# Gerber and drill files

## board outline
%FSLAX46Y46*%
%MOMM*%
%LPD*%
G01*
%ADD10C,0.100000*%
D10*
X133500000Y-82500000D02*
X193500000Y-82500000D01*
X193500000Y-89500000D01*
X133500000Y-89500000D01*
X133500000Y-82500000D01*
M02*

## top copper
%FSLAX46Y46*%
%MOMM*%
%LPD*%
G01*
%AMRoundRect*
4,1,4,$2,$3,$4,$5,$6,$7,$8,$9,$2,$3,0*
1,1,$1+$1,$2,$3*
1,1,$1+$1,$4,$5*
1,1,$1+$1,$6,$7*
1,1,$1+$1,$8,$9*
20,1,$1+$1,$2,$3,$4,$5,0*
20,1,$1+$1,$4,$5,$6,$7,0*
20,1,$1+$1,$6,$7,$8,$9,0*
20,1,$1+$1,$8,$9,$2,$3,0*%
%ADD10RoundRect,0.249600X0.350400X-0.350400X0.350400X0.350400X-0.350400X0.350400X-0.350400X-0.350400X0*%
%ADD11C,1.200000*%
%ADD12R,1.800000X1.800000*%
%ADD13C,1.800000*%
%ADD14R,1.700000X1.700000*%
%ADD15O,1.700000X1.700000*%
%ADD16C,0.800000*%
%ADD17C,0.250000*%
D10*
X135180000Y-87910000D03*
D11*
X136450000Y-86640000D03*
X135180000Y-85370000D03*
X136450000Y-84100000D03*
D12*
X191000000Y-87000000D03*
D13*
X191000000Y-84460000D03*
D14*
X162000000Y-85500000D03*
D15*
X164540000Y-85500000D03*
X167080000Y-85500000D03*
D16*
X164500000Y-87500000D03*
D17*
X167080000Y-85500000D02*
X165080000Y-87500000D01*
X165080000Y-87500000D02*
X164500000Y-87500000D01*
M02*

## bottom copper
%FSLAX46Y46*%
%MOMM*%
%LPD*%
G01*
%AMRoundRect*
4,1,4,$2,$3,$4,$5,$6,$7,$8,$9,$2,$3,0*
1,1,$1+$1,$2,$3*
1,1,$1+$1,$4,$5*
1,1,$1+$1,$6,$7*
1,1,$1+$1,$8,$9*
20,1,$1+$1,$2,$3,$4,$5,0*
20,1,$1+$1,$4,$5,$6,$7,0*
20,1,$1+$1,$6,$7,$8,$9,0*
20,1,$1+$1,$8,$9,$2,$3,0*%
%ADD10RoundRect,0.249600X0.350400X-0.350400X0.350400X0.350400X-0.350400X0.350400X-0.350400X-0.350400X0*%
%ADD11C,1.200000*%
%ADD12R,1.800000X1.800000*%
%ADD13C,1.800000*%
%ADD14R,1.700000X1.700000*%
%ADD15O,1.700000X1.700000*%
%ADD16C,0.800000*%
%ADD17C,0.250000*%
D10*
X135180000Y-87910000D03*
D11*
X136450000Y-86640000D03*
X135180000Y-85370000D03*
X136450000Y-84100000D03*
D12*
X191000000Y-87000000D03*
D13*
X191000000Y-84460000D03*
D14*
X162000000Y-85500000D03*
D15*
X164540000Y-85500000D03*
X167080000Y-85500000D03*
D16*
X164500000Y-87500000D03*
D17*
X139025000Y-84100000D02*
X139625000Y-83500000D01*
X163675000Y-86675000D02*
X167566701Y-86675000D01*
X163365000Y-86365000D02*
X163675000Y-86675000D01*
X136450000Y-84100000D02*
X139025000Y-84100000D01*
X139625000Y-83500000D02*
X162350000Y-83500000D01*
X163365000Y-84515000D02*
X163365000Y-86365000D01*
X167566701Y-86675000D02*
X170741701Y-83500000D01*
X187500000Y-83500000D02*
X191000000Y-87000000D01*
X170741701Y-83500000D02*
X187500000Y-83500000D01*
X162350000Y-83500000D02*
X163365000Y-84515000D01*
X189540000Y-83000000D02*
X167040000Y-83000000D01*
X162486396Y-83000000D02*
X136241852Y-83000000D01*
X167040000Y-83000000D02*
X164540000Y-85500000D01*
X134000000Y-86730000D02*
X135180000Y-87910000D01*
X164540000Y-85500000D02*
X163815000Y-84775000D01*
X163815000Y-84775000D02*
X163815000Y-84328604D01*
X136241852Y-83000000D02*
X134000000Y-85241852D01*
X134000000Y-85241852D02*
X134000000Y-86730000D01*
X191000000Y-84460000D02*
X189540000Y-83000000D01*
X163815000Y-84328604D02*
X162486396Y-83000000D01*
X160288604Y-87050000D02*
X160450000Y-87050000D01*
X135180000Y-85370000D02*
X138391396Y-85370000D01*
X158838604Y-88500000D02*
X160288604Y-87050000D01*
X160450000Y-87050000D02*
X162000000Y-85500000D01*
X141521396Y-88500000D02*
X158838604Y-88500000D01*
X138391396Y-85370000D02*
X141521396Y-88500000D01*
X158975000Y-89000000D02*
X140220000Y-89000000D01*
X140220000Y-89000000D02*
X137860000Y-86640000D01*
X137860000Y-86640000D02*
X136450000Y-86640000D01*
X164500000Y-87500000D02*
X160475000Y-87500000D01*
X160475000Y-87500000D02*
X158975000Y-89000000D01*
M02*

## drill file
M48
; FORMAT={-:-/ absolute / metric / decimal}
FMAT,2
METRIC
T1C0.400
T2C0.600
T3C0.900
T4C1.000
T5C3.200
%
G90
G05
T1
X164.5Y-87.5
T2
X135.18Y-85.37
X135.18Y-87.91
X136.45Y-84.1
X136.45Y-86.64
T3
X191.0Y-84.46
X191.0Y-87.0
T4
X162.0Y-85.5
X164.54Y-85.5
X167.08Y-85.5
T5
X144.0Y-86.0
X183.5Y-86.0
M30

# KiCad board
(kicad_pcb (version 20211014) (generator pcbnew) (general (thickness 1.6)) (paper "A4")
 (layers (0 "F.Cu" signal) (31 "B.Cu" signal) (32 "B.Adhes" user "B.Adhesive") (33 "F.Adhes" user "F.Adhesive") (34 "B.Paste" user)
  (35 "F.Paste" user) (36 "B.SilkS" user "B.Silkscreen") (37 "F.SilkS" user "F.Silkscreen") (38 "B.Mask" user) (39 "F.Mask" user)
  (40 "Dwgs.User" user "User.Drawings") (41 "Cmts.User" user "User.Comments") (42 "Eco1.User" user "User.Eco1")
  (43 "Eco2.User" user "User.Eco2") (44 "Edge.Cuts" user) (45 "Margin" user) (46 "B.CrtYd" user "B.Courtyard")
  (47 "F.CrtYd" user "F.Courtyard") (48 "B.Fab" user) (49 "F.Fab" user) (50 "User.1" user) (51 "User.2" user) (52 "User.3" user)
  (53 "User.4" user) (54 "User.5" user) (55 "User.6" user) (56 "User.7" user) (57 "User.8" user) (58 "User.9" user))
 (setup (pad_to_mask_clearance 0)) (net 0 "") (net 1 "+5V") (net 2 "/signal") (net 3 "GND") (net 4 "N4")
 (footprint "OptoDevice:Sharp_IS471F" (layer "F.Cu") (at 135.18 87.91 90)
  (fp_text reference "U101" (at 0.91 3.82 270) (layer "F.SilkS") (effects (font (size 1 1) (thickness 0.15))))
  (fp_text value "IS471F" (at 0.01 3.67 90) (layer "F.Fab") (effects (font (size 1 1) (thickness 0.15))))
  (pad "1" thru_hole roundrect (at 0 0 90) (size 1.2 1.2) (drill 0.6) (layers *.Cu *.Mask) (roundrect_rratio 0.208) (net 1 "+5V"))
  (pad "2" thru_hole circle (at 1.27 1.27 90) (size 1.2 1.2) (drill 0.6) (layers *.Cu *.Mask) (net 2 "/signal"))
  (pad "3" thru_hole circle (at 2.54 0 90) (size 1.2 1.2) (drill 0.6) (layers *.Cu *.Mask) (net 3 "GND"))
  (pad "4" thru_hole circle (at 3.81 1.27 90) (size 1.2 1.2) (drill 0.6) (layers *.Cu *.Mask) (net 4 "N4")))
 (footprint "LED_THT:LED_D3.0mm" (layer "F.Cu") (at 191 87 90)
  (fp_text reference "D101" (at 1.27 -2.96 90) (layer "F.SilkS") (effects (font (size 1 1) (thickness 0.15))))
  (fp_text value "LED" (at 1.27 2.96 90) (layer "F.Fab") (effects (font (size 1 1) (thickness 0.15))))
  (pad "1" thru_hole rect (at 0 0 90) (size 1.8 1.8) (drill 0.9) (layers *.Cu *.Mask) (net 4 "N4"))
  (pad "2" thru_hole circle (at 2.54 0 90) (size 1.8 1.8) (drill 0.9) (layers *.Cu *.Mask) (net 1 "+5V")))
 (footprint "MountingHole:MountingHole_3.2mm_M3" (layer "F.Cu") (at 183.5 86)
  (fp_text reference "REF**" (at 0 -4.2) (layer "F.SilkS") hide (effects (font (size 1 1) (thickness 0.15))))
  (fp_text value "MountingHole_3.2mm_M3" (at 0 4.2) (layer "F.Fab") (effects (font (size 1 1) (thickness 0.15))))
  (pad "" np_thru_hole circle (at 0 0) (size 3.2 3.2) (drill 3.2) (layers F&B.Cu *.Mask)))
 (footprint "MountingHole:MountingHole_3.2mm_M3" (layer "F.Cu") (at 144 86)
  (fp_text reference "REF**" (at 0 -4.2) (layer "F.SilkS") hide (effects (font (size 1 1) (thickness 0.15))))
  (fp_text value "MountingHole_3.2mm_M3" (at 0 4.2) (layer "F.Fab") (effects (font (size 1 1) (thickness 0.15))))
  (pad "" np_thru_hole circle (at 0 0) (size 3.2 3.2) (drill 3.2) (layers *.Cu *.Mask)))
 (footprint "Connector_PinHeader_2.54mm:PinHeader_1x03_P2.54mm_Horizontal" (layer "B.Cu") (at 162 85.5 -90)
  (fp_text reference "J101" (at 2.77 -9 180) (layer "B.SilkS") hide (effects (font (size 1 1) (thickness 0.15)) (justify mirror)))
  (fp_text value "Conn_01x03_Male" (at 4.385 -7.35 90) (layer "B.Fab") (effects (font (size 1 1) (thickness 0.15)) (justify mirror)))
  (pad "1" thru_hole rect (at 0 0 270) (size 1.7 1.7) (drill 1) (layers *.Cu *.Mask) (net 3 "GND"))
  (pad "2" thru_hole oval (at 0 -2.54 270) (size 1.7 1.7) (drill 1) (layers *.Cu *.Mask) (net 1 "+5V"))
  (pad "3" thru_hole oval (at 0 -5.08 270) (size 1.7 1.7) (drill 1) (layers *.Cu *.Mask) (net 2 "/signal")))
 (gr_rect (start 133.5 82.5) (end 193.5 89.5) (layer "Edge.Cuts") (width 0.1) (fill none))
 (segment (start 139.025 84.1) (end 139.625 83.5) (width 0.25) (layer "B.Cu") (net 4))
 (segment (start 163.675 86.675) (end 167.566701 86.675) (width 0.25) (layer "B.Cu") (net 4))
 (segment (start 163.365 86.365) (end 163.675 86.675) (width 0.25) (layer "B.Cu") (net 4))
 (segment (start 136.45 84.1) (end 139.025 84.1) (width 0.25) (layer "B.Cu") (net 4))
 (segment (start 139.625 83.5) (end 162.35 83.5) (width 0.25) (layer "B.Cu") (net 4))
 (segment (start 163.365 84.515) (end 163.365 86.365) (width 0.25) (layer "B.Cu") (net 4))
 (segment (start 167.566701 86.675) (end 170.741701 83.5) (width 0.25) (layer "B.Cu") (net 4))
 (segment (start 187.5 83.5) (end 191 87) (width 0.25) (layer "B.Cu") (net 4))
 (segment (start 170.741701 83.5) (end 187.5 83.5) (width 0.25) (layer "B.Cu") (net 4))
 (segment (start 162.35 83.5) (end 163.365 84.515) (width 0.25) (layer "B.Cu") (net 4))
 (segment (start 189.54 83) (end 167.04 83) (width 0.25) (layer "B.Cu") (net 1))
 (segment (start 162.486396 83) (end 136.241852 83) (width 0.25) (layer "B.Cu") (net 1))
 (segment (start 167.04 83) (end 164.54 85.5) (width 0.25) (layer "B.Cu") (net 1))
 (segment (start 134 86.73) (end 135.18 87.91) (width 0.25) (layer "B.Cu") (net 1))
 (segment (start 164.54 85.5) (end 163.815 84.775) (width 0.25) (layer "B.Cu") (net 1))
 (segment (start 163.815 84.775) (end 163.815 84.328604) (width 0.25) (layer "B.Cu") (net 1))
 (segment (start 136.241852 83) (end 134 85.241852) (width 0.25) (layer "B.Cu") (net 1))
 (segment (start 134 85.241852) (end 134 86.73) (width 0.25) (layer "B.Cu") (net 1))
 (segment (start 191 84.46) (end 189.54 83) (width 0.25) (layer "B.Cu") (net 1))
 (segment (start 163.815 84.328604) (end 162.486396 83) (width 0.25) (layer "B.Cu") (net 1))
 (segment (start 160.288604 87.05) (end 160.45 87.05) (width 0.25) (layer "B.Cu") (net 3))
 (segment (start 135.18 85.37) (end 138.391396 85.37) (width 0.25) (layer "B.Cu") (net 3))
 (segment (start 158.838604 88.5) (end 160.288604 87.05) (width 0.25) (layer "B.Cu") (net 3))
 (segment (start 160.45 87.05) (end 162 85.5) (width 0.25) (layer "B.Cu") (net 3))
 (segment (start 141.521396 88.5) (end 158.838604 88.5) (width 0.25) (layer "B.Cu") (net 3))
 (segment (start 138.391396 85.37) (end 141.521396 88.5) (width 0.25) (layer "B.Cu") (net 3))
 (segment (start 167.08 85.5) (end 165.08 87.5) (width 0.25) (layer "F.Cu") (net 2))
 (segment (start 165.08 87.5) (end 164.5 87.5) (width 0.25) (layer "F.Cu") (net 2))
 (via (at 164.5 87.5) (size 0.8) (drill 0.4) (layers "F.Cu" "B.Cu") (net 2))
 (segment (start 158.975 89) (end 140.22 89) (width 0.25) (layer "B.Cu") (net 2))
 (segment (start 140.22 89) (end 137.86 86.64) (width 0.25) (layer "B.Cu") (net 2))
 (segment (start 137.86 86.64) (end 136.45 86.64) (width 0.25) (layer "B.Cu") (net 2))
 (segment (start 164.5 87.5) (end 160.475 87.5) (width 0.25) (layer "B.Cu") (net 2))
 (segment (start 160.475 87.5) (end 158.975 89) (width 0.25) (layer "B.Cu") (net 2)))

